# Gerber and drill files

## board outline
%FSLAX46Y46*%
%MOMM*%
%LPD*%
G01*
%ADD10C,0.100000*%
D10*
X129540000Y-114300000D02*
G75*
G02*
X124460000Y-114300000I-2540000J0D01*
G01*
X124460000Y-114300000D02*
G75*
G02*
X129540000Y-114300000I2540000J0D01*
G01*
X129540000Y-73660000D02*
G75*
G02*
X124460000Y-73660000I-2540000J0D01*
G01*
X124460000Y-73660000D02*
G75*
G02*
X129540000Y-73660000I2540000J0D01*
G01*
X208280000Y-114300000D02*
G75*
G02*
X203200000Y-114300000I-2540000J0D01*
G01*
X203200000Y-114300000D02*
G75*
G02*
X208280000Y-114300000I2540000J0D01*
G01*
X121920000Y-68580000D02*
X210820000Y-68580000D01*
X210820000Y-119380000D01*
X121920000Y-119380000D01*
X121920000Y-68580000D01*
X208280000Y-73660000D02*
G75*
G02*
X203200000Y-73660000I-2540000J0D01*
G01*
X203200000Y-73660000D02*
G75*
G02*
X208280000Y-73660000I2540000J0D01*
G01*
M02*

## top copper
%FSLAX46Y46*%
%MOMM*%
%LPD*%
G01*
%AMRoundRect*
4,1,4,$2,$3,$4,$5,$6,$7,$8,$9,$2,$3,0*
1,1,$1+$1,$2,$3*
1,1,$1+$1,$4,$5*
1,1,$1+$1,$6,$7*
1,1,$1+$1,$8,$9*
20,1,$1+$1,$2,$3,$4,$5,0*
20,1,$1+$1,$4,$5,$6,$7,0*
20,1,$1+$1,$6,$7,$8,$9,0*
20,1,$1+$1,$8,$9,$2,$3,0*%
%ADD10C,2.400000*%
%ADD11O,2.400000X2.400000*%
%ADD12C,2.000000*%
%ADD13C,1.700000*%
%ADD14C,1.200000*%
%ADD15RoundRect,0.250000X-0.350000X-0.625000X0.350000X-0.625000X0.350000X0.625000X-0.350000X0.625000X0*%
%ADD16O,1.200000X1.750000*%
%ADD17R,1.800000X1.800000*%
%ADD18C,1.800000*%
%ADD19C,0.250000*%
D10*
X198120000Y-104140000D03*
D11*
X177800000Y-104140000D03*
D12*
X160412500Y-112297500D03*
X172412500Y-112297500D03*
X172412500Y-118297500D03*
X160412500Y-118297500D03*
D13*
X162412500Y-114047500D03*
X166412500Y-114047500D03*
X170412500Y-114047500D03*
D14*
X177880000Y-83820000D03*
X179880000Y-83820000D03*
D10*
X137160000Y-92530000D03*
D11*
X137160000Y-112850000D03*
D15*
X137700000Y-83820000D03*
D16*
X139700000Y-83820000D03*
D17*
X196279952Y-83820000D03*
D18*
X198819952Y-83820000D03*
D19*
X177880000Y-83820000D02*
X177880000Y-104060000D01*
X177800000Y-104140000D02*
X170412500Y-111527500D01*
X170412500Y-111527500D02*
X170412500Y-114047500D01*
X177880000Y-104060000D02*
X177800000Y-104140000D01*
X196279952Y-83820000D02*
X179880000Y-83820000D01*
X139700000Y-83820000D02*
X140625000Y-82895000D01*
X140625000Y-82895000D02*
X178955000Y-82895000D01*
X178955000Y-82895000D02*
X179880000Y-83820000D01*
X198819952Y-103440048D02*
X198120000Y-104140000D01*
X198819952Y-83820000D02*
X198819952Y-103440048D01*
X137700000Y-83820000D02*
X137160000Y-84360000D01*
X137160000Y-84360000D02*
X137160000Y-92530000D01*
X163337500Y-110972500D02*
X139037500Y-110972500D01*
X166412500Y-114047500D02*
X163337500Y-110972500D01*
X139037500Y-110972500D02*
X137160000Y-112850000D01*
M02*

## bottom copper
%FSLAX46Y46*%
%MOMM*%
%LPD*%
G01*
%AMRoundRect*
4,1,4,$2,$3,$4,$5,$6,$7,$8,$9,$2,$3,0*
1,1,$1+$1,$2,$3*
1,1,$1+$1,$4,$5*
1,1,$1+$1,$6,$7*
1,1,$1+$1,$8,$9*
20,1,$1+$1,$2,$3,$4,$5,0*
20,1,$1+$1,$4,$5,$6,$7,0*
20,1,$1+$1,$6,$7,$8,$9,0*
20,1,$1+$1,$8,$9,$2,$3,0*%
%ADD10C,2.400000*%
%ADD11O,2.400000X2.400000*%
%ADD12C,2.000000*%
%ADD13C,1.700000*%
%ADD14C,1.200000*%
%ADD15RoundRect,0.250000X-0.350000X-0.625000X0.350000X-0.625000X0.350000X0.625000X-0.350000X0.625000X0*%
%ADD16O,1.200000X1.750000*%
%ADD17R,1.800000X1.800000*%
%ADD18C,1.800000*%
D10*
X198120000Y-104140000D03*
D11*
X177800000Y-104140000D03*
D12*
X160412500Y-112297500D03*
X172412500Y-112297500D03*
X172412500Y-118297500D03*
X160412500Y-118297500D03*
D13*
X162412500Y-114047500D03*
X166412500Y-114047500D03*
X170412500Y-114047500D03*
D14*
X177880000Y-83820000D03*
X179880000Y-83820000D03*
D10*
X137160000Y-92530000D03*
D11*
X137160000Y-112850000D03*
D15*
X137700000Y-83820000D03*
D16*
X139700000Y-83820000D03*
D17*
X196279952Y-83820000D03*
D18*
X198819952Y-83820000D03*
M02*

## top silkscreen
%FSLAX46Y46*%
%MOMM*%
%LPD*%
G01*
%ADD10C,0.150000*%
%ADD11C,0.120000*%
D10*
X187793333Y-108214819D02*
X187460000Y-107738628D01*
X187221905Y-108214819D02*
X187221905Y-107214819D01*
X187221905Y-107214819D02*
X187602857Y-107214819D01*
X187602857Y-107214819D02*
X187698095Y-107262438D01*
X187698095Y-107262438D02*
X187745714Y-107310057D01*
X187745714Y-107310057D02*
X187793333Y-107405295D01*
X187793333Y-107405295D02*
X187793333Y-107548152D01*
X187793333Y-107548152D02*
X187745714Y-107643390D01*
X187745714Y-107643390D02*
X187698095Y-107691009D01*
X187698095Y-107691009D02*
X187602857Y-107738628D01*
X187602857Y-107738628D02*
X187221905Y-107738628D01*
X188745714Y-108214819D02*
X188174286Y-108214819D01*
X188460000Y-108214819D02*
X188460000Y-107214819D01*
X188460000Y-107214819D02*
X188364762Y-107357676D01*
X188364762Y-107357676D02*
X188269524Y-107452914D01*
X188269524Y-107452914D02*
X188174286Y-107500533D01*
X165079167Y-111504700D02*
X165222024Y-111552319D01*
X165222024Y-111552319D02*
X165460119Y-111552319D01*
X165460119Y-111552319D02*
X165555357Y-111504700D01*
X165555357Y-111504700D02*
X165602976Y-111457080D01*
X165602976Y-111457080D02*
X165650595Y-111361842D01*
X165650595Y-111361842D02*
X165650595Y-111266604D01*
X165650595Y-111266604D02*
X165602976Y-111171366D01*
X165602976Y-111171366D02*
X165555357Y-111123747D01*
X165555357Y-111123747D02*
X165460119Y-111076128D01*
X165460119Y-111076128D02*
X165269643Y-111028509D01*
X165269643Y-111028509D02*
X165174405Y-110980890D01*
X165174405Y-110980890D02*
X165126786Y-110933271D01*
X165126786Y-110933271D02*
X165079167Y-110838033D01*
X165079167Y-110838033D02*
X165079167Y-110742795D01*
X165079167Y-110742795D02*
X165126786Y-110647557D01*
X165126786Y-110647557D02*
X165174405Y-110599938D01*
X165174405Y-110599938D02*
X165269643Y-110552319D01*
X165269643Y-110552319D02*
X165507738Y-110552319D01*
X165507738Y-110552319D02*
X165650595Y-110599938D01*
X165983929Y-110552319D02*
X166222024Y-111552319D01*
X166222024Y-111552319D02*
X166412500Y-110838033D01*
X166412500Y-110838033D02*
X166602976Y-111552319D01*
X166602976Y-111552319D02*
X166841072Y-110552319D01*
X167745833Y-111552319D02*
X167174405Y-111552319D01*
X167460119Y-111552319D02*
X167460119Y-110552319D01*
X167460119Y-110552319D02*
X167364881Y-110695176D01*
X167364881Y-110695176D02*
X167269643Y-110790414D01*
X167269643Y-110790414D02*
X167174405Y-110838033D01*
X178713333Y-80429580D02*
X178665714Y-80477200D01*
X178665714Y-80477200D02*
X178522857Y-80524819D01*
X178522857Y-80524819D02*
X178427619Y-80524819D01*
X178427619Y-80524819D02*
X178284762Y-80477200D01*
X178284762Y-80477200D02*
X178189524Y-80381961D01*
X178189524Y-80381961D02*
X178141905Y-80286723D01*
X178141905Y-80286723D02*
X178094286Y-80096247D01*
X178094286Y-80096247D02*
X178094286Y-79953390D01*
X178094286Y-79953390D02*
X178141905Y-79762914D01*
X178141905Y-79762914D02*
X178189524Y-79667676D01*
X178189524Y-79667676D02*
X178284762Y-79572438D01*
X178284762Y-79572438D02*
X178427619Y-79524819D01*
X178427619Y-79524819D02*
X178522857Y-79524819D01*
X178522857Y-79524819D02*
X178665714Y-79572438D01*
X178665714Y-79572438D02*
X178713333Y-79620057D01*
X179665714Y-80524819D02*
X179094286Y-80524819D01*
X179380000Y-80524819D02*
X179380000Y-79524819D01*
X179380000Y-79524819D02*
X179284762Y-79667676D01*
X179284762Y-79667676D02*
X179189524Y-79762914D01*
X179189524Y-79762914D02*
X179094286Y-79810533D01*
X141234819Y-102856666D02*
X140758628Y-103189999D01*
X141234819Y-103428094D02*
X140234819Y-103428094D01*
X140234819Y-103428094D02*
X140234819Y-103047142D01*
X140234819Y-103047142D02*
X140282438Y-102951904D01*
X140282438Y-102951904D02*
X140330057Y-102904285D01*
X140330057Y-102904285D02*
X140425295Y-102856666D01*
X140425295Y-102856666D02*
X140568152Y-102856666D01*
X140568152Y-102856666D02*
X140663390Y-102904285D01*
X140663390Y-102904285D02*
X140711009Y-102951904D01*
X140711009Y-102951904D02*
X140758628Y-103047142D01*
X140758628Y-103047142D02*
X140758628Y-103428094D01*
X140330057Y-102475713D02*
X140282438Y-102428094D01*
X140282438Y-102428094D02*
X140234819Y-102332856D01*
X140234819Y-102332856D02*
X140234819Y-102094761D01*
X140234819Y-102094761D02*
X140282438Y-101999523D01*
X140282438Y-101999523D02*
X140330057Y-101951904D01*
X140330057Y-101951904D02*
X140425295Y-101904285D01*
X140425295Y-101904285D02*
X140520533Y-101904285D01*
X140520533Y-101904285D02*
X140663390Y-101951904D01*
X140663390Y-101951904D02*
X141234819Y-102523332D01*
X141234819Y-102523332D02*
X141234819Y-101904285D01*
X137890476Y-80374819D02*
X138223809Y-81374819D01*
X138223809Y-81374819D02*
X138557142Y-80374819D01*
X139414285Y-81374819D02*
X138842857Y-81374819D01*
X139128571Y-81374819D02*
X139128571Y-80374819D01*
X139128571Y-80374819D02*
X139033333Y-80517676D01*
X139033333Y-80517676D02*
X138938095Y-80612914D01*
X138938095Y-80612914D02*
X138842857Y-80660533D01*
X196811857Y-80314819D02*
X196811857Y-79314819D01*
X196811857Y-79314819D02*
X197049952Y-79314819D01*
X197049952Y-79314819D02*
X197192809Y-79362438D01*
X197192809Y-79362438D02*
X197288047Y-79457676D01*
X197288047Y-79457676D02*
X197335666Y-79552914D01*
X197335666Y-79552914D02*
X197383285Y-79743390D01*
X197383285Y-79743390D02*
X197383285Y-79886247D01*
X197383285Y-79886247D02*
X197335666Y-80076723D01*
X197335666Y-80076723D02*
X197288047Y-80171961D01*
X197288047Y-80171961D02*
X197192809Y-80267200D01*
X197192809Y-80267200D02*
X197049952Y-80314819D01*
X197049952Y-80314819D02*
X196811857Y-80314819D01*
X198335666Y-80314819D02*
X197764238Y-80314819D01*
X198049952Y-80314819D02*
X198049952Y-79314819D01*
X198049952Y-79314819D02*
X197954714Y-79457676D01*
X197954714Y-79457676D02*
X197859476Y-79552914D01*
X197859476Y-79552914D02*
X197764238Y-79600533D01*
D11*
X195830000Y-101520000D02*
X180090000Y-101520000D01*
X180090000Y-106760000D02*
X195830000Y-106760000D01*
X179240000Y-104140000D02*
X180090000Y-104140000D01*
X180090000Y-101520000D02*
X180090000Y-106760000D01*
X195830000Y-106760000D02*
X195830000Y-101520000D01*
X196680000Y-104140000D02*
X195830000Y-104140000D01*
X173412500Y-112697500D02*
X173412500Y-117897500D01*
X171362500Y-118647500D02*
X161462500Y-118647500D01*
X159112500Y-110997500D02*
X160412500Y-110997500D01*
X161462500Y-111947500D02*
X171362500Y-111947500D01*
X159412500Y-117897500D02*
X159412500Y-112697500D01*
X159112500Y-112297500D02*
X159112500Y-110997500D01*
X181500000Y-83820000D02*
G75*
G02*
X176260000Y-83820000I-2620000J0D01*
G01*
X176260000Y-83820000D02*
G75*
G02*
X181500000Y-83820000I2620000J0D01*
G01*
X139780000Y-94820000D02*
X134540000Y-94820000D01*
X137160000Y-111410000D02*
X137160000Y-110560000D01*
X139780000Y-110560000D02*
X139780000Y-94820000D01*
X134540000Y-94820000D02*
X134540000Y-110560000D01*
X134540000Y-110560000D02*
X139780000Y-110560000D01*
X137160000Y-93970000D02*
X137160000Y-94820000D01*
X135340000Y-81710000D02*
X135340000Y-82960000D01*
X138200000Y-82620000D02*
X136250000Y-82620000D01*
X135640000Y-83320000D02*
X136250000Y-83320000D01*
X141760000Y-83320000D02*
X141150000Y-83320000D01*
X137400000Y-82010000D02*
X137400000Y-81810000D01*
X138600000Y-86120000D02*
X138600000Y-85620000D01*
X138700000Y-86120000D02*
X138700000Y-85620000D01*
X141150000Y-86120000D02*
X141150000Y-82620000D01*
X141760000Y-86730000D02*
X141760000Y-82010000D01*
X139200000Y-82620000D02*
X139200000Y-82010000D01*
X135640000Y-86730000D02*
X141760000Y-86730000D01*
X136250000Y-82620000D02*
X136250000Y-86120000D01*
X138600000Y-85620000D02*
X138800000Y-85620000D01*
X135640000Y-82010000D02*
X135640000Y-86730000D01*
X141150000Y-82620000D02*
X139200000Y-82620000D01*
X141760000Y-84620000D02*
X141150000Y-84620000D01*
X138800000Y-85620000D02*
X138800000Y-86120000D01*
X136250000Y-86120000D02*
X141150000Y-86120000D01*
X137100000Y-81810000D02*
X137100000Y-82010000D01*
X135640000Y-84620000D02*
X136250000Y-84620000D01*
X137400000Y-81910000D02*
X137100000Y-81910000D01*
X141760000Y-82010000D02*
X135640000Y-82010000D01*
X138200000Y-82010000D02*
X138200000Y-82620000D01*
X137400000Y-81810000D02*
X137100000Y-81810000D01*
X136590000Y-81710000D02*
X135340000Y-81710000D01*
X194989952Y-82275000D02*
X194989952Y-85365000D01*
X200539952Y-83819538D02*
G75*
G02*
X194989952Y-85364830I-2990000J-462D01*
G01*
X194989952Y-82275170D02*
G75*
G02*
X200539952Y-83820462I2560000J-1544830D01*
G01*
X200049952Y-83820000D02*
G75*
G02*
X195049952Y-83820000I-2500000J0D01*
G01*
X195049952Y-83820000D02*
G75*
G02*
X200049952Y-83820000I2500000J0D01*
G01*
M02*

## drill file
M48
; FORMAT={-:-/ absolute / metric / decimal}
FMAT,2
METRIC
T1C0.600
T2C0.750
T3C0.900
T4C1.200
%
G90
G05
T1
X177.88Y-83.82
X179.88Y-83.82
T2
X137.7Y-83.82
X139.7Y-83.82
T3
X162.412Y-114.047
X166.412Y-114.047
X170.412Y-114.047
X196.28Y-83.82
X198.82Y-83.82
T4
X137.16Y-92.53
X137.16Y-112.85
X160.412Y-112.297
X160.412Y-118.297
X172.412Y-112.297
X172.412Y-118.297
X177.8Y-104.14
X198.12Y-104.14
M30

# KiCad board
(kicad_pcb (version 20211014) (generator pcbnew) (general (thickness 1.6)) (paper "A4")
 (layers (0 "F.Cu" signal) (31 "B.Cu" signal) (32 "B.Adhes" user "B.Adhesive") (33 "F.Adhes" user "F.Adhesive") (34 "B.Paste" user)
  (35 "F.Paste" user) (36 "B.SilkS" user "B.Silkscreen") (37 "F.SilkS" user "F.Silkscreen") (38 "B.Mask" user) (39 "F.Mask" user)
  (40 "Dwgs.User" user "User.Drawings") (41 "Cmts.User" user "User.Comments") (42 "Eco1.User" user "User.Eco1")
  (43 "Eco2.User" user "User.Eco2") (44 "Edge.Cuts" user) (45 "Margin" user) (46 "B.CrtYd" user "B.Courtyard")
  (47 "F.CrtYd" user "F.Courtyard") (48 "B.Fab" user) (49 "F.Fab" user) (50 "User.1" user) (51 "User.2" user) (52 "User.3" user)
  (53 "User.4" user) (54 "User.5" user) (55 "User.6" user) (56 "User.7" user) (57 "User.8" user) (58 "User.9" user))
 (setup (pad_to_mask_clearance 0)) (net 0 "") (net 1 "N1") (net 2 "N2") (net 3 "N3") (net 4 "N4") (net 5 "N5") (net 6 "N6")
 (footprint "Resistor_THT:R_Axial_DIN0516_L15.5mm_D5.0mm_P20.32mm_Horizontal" (layer "F.Cu") (at 198.12 104.14 180)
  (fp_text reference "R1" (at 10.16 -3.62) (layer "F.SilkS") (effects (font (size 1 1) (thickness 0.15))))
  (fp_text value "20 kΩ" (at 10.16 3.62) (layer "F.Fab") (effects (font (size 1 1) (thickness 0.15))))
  (fp_line (start 2.29 2.62) (end 18.03 2.62) (layer "F.SilkS") (width 0.12))
  (fp_line (start 18.03 -2.62) (end 2.29 -2.62) (layer "F.SilkS") (width 0.12))
  (fp_line (start 18.88 0) (end 18.03 0) (layer "F.SilkS") (width 0.12))
  (fp_line (start 18.03 2.62) (end 18.03 -2.62) (layer "F.SilkS") (width 0.12))
  (fp_line (start 2.29 -2.62) (end 2.29 2.62) (layer "F.SilkS") (width 0.12))
  (fp_line (start 1.44 0) (end 2.29 0) (layer "F.SilkS") (width 0.12))
  (pad "1" thru_hole circle (at 0 0 180) (size 2.4 2.4) (drill 1.2) (layers *.Cu *.Mask) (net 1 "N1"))
  (pad "2" thru_hole oval (at 20.32 0 180) (size 2.4 2.4) (drill 1.2) (layers *.Cu *.Mask) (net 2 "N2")))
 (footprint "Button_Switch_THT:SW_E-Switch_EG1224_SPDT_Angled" (layer "F.Cu") (at 162.4125 114.0475)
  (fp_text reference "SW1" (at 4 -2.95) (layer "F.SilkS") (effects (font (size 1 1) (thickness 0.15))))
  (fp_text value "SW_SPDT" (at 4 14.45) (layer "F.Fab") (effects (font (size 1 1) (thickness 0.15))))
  (fp_line (start 11 -1.35) (end 11 3.85) (layer "F.SilkS") (width 0.12))
  (fp_line (start 8.95 4.6) (end -0.95 4.6) (layer "F.SilkS") (width 0.12))
  (fp_line (start -3.3 -3.05) (end -2 -3.05) (layer "F.SilkS") (width 0.12))
  (fp_line (start -0.95 -2.1) (end 8.95 -2.1) (layer "F.SilkS") (width 0.12))
  (fp_line (start -3 3.85) (end -3 -1.35) (layer "F.SilkS") (width 0.12))
  (fp_line (start -3.3 -1.75) (end -3.3 -3.05) (layer "F.SilkS") (width 0.12))
  (pad "" thru_hole circle (at -2 -1.75) (size 2 2) (drill 1.2) (layers *.Cu *.Mask))
  (pad "" thru_hole circle (at 10 -1.75) (size 2 2) (drill 1.2) (layers *.Cu *.Mask))
  (pad "" thru_hole circle (at 10 4.25) (size 2 2) (drill 1.2) (layers *.Cu *.Mask))
  (pad "" thru_hole circle (at -2 4.25) (size 2 2) (drill 1.2) (layers *.Cu *.Mask))
  (pad "1" thru_hole circle (at 0 0) (size 1.7 1.7) (drill 0.9) (layers *.Cu *.Mask) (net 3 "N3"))
  (pad "2" thru_hole circle (at 4 0) (size 1.7 1.7) (drill 0.9) (layers *.Cu *.Mask) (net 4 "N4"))
  (pad "3" thru_hole circle (at 8 0) (size 1.7 1.7) (drill 0.9) (layers *.Cu *.Mask) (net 2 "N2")))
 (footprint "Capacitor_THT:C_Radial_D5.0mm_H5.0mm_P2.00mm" (layer "F.Cu") (at 177.88 83.82)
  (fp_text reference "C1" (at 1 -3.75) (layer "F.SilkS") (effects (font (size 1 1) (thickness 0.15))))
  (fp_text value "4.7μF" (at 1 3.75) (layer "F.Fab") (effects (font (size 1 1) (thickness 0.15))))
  (fp_circle (center 1 0) (end 3.62 0) (layer "F.SilkS") (width 0.12) (fill none))
  (pad "1" thru_hole circle (at 0 0) (size 1.2 1.2) (drill 0.6) (layers *.Cu *.Mask) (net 2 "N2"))
  (pad "2" thru_hole circle (at 2 0) (size 1.2 1.2) (drill 0.6) (layers *.Cu *.Mask) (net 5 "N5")))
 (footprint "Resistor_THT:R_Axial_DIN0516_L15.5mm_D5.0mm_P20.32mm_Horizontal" (layer "F.Cu") (at 137.16 92.53 -90)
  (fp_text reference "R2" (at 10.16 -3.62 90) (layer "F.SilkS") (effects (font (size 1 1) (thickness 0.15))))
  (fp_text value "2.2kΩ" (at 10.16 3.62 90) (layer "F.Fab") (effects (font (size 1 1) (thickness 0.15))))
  (fp_line (start 2.29 -2.62) (end 2.29 2.62) (layer "F.SilkS") (width 0.12))
  (fp_line (start 18.88 0) (end 18.03 0) (layer "F.SilkS") (width 0.12))
  (fp_line (start 18.03 -2.62) (end 2.29 -2.62) (layer "F.SilkS") (width 0.12))
  (fp_line (start 2.29 2.62) (end 18.03 2.62) (layer "F.SilkS") (width 0.12))
  (fp_line (start 18.03 2.62) (end 18.03 -2.62) (layer "F.SilkS") (width 0.12))
  (fp_line (start 1.44 0) (end 2.29 0) (layer "F.SilkS") (width 0.12))
  (pad "1" thru_hole circle (at 0 0 270) (size 2.4 2.4) (drill 1.2) (layers *.Cu *.Mask) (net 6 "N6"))
  (pad "2" thru_hole oval (at 20.32 0 270) (size 2.4 2.4) (drill 1.2) (layers *.Cu *.Mask) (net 4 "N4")))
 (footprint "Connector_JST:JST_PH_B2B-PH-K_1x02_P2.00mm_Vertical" (layer "F.Cu") (at 137.7 83.82)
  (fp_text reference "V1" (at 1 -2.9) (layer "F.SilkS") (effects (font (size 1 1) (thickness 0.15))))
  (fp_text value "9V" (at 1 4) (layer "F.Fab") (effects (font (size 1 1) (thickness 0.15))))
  (fp_line (start -2.36 -2.11) (end -2.36 -0.86) (layer "F.SilkS") (width 0.12))
  (fp_line (start 0.5 -1.2) (end -1.45 -1.2) (layer "F.SilkS") (width 0.12))
  (fp_line (start -2.06 -0.5) (end -1.45 -0.5) (layer "F.SilkS") (width 0.12))
  (fp_line (start 4.06 -0.5) (end 3.45 -0.5) (layer "F.SilkS") (width 0.12))
  (fp_line (start -0.3 -1.81) (end -0.3 -2.01) (layer "F.SilkS") (width 0.12))
  (fp_line (start 0.9 2.3) (end 0.9 1.8) (layer "F.SilkS") (width 0.12))
  (fp_line (start 1 2.3) (end 1 1.8) (layer "F.SilkS") (width 0.12))
  (fp_line (start 3.45 2.3) (end 3.45 -1.2) (layer "F.SilkS") (width 0.12))
  (fp_line (start 4.06 2.91) (end 4.06 -1.81) (layer "F.SilkS") (width 0.12))
  (fp_line (start 1.5 -1.2) (end 1.5 -1.81) (layer "F.SilkS") (width 0.12))
  (fp_line (start -2.06 2.91) (end 4.06 2.91) (layer "F.SilkS") (width 0.12))
  (fp_line (start -1.45 -1.2) (end -1.45 2.3) (layer "F.SilkS") (width 0.12))
  (fp_line (start 0.9 1.8) (end 1.1 1.8) (layer "F.SilkS") (width 0.12))
  (fp_line (start -2.06 -1.81) (end -2.06 2.91) (layer "F.SilkS") (width 0.12))
  (fp_line (start 3.45 -1.2) (end 1.5 -1.2) (layer "F.SilkS") (width 0.12))
  (fp_line (start 4.06 0.8) (end 3.45 0.8) (layer "F.SilkS") (width 0.12))
  (fp_line (start 1.1 1.8) (end 1.1 2.3) (layer "F.SilkS") (width 0.12))
  (fp_line (start -1.45 2.3) (end 3.45 2.3) (layer "F.SilkS") (width 0.12))
  (fp_line (start -0.6 -2.01) (end -0.6 -1.81) (layer "F.SilkS") (width 0.12))
  (fp_line (start -2.06 0.8) (end -1.45 0.8) (layer "F.SilkS") (width 0.12))
  (fp_line (start -0.3 -1.91) (end -0.6 -1.91) (layer "F.SilkS") (width 0.12))
  (fp_line (start 4.06 -1.81) (end -2.06 -1.81) (layer "F.SilkS") (width 0.12))
  (fp_line (start 0.5 -1.81) (end 0.5 -1.2) (layer "F.SilkS") (width 0.12))
  (fp_line (start -0.3 -2.01) (end -0.6 -2.01) (layer "F.SilkS") (width 0.12))
  (fp_line (start -1.11 -2.11) (end -2.36 -2.11) (layer "F.SilkS") (width 0.12))
  (pad "1" thru_hole roundrect (at 0 0) (size 1.2 1.75) (drill 0.75) (layers *.Cu *.Mask) (roundrect_rratio 0.208333) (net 6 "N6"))
  (pad "2" thru_hole oval (at 2 0) (size 1.2 1.75) (drill 0.75) (layers *.Cu *.Mask) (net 5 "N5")))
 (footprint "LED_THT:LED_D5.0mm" (layer "F.Cu") (at 196.279952 83.82)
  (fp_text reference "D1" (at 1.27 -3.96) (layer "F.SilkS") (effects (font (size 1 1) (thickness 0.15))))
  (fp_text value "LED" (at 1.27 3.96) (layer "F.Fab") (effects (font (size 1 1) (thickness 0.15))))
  (fp_line (start -1.29 -1.545) (end -1.29 1.545) (layer "F.SilkS") (width 0.12))
  (fp_arc (start 4.26 -0.000462) (mid 2.072002 2.880433) (end -1.29 1.54483) (layer "F.SilkS") (width 0.12))
  (fp_arc (start -1.29 -1.54483) (mid 2.072002 -2.880433) (end 4.26 0.000462) (layer "F.SilkS") (width 0.12))
  (fp_circle (center 1.27 0) (end 3.77 0) (layer "F.SilkS") (width 0.12) (fill none))
  (pad "1" thru_hole rect (at 0 0) (size 1.8 1.8) (drill 0.9) (layers *.Cu *.Mask) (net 5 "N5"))
  (pad "2" thru_hole circle (at 2.54 0) (size 1.8 1.8) (drill 0.9) (layers *.Cu *.Mask) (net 1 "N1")))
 (gr_circle (center 127 114.3) (end 127 116.84) (layer "Edge.Cuts") (width 0.1) (fill none))
 (gr_circle (center 127 73.66) (end 127 76.2) (layer "Edge.Cuts") (width 0.1) (fill none))
 (gr_circle (center 205.74 114.3) (end 205.74 116.84) (layer "Edge.Cuts") (width 0.1) (fill none))
 (gr_rect (start 121.92 68.58) (end 210.82 119.38) (layer "Edge.Cuts") (width 0.1) (fill none))
 (gr_circle (center 205.74 73.66) (end 205.74 76.2) (layer "Edge.Cuts") (width 0.1) (fill none))
 (segment (start 177.88 83.82) (end 177.88 104.06) (width 0.25) (layer "F.Cu") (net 2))
 (segment (start 177.8 104.14) (end 170.4125 111.5275) (width 0.25) (layer "F.Cu") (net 2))
 (segment (start 170.4125 111.5275) (end 170.4125 114.0475) (width 0.25) (layer "F.Cu") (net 2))
 (segment (start 177.88 104.06) (end 177.8 104.14) (width 0.25) (layer "F.Cu") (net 2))
 (segment (start 196.279952 83.82) (end 179.88 83.82) (width 0.25) (layer "F.Cu") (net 5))
 (segment (start 139.7 83.82) (end 140.625 82.895) (width 0.25) (layer "F.Cu") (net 5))
 (segment (start 140.625 82.895) (end 178.955 82.895) (width 0.25) (layer "F.Cu") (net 5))
 (segment (start 178.955 82.895) (end 179.88 83.82) (width 0.25) (layer "F.Cu") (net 5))
 (segment (start 198.819952 103.440048) (end 198.12 104.14) (width 0.25) (layer "F.Cu") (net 1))
 (segment (start 198.819952 83.82) (end 198.819952 103.440048) (width 0.25) (layer "F.Cu") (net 1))
 (segment (start 137.7 83.82) (end 137.16 84.36) (width 0.25) (layer "F.Cu") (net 6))
 (segment (start 137.16 84.36) (end 137.16 92.53) (width 0.25) (layer "F.Cu") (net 6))
 (segment (start 163.3375 110.9725) (end 139.0375 110.9725) (width 0.25) (layer "F.Cu") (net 4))
 (segment (start 166.4125 114.0475) (end 163.3375 110.9725) (width 0.25) (layer "F.Cu") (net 4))
 (segment (start 139.0375 110.9725) (end 137.16 112.85) (width 0.25) (layer "F.Cu") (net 4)))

